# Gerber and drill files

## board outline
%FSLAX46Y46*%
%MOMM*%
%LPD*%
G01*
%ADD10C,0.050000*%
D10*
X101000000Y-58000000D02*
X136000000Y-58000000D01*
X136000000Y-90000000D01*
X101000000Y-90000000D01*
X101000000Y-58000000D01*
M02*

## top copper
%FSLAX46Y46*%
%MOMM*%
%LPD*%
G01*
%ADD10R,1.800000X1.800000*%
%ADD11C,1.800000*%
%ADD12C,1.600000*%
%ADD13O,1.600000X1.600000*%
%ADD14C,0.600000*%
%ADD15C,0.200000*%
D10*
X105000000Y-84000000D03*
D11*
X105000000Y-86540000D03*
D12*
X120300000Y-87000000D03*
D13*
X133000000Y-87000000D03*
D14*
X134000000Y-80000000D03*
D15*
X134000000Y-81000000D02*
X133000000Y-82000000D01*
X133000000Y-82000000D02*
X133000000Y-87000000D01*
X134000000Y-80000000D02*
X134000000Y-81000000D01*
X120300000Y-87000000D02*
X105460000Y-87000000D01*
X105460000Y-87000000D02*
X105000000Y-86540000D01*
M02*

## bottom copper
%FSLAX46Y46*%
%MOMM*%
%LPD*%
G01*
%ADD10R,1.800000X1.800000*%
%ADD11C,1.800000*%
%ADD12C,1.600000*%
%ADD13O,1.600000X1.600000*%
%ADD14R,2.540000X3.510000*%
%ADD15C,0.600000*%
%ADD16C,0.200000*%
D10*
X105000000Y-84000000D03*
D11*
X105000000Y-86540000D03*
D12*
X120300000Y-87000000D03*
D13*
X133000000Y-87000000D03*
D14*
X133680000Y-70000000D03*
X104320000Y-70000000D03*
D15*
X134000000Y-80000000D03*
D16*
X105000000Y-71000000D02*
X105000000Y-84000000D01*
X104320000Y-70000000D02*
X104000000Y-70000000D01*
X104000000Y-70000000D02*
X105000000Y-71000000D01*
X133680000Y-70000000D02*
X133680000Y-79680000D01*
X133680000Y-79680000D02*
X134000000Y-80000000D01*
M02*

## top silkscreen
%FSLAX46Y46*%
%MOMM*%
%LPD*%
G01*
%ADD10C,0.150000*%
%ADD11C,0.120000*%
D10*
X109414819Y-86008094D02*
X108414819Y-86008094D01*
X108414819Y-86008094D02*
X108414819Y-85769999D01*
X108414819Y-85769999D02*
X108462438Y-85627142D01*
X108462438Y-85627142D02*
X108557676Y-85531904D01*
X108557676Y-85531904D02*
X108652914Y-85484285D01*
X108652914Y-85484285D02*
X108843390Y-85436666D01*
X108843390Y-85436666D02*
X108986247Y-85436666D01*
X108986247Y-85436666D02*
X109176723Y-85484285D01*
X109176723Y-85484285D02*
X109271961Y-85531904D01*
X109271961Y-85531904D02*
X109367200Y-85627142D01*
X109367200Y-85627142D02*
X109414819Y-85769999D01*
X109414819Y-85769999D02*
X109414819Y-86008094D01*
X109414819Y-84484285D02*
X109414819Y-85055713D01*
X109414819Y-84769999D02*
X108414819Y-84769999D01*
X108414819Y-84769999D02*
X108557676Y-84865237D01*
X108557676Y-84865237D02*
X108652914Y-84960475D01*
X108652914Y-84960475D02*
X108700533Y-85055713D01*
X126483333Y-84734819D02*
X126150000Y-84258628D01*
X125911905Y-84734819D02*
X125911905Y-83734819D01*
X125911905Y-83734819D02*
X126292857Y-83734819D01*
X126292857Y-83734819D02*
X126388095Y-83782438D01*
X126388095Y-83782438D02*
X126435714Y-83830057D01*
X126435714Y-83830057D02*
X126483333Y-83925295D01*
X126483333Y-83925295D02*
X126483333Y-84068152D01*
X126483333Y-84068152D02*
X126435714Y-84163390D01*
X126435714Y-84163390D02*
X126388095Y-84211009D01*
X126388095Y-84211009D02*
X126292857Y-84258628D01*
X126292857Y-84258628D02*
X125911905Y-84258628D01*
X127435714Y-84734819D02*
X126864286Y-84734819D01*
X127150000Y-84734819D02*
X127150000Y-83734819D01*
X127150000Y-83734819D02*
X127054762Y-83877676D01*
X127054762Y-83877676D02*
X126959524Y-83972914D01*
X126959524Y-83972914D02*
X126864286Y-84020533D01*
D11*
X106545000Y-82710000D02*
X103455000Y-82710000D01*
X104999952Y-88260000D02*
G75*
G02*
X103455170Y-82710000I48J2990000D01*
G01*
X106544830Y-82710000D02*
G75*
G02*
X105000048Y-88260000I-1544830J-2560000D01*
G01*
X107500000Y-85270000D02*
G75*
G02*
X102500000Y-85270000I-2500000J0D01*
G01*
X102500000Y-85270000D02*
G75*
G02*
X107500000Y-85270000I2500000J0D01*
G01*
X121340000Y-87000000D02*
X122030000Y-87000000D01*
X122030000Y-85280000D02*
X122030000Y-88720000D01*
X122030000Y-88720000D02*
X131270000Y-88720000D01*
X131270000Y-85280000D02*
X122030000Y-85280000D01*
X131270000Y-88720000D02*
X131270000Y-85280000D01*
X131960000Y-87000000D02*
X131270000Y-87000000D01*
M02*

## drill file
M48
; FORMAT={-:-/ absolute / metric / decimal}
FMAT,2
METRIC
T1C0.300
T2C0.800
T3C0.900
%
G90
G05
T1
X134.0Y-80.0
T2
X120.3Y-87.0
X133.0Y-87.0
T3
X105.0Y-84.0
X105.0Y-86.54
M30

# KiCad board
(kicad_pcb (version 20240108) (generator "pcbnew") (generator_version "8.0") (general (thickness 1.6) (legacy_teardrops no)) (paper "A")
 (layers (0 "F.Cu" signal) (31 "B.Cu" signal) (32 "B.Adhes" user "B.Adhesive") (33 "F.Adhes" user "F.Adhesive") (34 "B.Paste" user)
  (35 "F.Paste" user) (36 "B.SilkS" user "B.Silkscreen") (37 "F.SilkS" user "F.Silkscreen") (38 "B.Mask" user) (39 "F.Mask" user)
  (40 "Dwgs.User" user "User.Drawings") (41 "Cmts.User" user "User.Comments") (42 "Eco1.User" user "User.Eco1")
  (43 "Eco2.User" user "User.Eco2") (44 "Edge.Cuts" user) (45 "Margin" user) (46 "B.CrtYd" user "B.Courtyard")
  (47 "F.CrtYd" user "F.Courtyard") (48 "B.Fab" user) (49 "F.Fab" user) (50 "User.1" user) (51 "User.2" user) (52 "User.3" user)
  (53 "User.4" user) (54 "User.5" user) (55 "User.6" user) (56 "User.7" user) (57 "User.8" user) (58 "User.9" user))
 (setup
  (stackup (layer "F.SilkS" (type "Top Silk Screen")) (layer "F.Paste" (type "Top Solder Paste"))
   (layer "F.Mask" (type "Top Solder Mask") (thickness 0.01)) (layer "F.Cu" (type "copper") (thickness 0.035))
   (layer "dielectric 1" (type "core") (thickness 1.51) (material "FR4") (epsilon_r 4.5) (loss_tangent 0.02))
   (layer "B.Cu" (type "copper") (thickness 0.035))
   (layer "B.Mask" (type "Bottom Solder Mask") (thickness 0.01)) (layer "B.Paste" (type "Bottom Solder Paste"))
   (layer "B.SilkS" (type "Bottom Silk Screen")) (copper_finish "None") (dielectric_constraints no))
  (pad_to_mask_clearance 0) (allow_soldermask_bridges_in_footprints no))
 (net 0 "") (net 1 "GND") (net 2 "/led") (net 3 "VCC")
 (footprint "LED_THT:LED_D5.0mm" (layer "F.Cu") (at 105 84 -90)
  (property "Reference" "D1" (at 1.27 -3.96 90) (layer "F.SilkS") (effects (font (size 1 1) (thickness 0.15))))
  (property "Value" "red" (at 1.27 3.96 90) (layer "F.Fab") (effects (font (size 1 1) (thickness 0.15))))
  (fp_line (start -1.29 -1.545) (end -1.29 1.545) (stroke (width 0.12) (type solid)) (layer "F.SilkS"))
  (fp_arc (start 4.26 0.000048) (mid 2.071756 2.880501) (end -1.29 1.54483) (stroke (width 0.12) (type solid)) (layer "F.SilkS"))
  (fp_arc (start -1.29 -1.54483) (mid 2.071756 -2.880501) (end 4.26 -0.000048) (stroke (width 0.12) (type solid)) (layer "F.SilkS"))
  (fp_circle (center 1.27 0) (end 3.77 0) (stroke (width 0.12) (type solid)) (fill none) (layer "F.SilkS"))
  (pad "1" thru_hole rect (at 0 0 270) (size 1.8 1.8) (drill 0.9) (layers "*.Cu" "*.Mask") (remove_unused_layers no) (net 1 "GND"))
  (pad "2" thru_hole circle (at 2.54 0 270) (size 1.8 1.8) (drill 0.9) (layers "*.Cu" "*.Mask") (remove_unused_layers no) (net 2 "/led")))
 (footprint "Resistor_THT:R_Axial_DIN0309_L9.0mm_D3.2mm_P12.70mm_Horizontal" (layer "F.Cu") (at 120.3 87)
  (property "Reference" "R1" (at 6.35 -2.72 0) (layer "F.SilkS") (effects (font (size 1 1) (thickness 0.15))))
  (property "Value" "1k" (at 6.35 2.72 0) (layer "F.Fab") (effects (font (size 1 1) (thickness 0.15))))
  (fp_line (start 1.04 0) (end 1.73 0) (stroke (width 0.12) (type solid)) (layer "F.SilkS"))
  (fp_line (start 1.73 -1.72) (end 1.73 1.72) (stroke (width 0.12) (type solid)) (layer "F.SilkS"))
  (fp_line (start 1.73 1.72) (end 10.97 1.72) (stroke (width 0.12) (type solid)) (layer "F.SilkS"))
  (fp_line (start 10.97 -1.72) (end 1.73 -1.72) (stroke (width 0.12) (type solid)) (layer "F.SilkS"))
  (fp_line (start 10.97 1.72) (end 10.97 -1.72) (stroke (width 0.12) (type solid)) (layer "F.SilkS"))
  (fp_line (start 11.66 0) (end 10.97 0) (stroke (width 0.12) (type solid)) (layer "F.SilkS"))
  (pad "1" thru_hole circle (at 0 0) (size 1.6 1.6) (drill 0.8) (layers "*.Cu" "*.Mask") (remove_unused_layers no) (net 2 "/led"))
  (pad "2" thru_hole oval (at 12.7 0) (size 1.6 1.6) (drill 0.8) (layers "*.Cu" "*.Mask") (remove_unused_layers no) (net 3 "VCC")))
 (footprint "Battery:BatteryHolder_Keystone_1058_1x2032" (layer "B.Cu") (at 119 70 180)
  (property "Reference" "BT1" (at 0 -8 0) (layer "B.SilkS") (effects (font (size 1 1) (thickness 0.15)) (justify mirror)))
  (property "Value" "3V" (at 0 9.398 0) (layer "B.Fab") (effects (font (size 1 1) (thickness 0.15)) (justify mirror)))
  (pad "1" smd rect (at -14.68 0 180) (size 2.54 3.51) (layers "B.Cu" "B.Paste" "B.Mask") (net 3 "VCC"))
  (pad "2" smd rect (at 14.68 0 180) (size 2.54 3.51) (layers "B.Cu" "B.Paste" "B.Mask") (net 1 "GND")))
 (gr_rect (start 101 58) (end 136 90) (stroke (width 0.05) (type default)) (fill none) (layer "Edge.Cuts"))
 (segment (start 105 71) (end 105 84) (width 0.2) (layer "B.Cu") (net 1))
 (segment (start 104.32 70) (end 104 70) (width 0.2) (layer "B.Cu") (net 1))
 (segment (start 104 70) (end 105 71) (width 0.2) (layer "B.Cu") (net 1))
 (segment (start 134 81) (end 133 82) (width 0.2) (layer "F.Cu") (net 3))
 (segment (start 133 82) (end 133 87) (width 0.2) (layer "F.Cu") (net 3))
 (segment (start 134 80) (end 134 81) (width 0.2) (layer "F.Cu") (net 3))
 (via (at 134 80) (size 0.6) (drill 0.3) (layers "F.Cu" "B.Cu") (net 3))
 (segment (start 133.68 70) (end 133.68 79.68) (width 0.2) (layer "B.Cu") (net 3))
 (segment (start 133.68 79.68) (end 134 80) (width 0.2) (layer "B.Cu") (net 3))
 (segment (start 120.3 87) (end 105.46 87) (width 0.2) (layer "F.Cu") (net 2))
 (segment (start 105.46 87) (end 105 86.54) (width 0.2) (layer "F.Cu") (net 2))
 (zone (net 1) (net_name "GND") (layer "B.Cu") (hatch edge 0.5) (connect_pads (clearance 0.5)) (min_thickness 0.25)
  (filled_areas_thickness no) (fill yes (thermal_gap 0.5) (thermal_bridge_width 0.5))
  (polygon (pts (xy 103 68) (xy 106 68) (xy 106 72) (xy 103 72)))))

